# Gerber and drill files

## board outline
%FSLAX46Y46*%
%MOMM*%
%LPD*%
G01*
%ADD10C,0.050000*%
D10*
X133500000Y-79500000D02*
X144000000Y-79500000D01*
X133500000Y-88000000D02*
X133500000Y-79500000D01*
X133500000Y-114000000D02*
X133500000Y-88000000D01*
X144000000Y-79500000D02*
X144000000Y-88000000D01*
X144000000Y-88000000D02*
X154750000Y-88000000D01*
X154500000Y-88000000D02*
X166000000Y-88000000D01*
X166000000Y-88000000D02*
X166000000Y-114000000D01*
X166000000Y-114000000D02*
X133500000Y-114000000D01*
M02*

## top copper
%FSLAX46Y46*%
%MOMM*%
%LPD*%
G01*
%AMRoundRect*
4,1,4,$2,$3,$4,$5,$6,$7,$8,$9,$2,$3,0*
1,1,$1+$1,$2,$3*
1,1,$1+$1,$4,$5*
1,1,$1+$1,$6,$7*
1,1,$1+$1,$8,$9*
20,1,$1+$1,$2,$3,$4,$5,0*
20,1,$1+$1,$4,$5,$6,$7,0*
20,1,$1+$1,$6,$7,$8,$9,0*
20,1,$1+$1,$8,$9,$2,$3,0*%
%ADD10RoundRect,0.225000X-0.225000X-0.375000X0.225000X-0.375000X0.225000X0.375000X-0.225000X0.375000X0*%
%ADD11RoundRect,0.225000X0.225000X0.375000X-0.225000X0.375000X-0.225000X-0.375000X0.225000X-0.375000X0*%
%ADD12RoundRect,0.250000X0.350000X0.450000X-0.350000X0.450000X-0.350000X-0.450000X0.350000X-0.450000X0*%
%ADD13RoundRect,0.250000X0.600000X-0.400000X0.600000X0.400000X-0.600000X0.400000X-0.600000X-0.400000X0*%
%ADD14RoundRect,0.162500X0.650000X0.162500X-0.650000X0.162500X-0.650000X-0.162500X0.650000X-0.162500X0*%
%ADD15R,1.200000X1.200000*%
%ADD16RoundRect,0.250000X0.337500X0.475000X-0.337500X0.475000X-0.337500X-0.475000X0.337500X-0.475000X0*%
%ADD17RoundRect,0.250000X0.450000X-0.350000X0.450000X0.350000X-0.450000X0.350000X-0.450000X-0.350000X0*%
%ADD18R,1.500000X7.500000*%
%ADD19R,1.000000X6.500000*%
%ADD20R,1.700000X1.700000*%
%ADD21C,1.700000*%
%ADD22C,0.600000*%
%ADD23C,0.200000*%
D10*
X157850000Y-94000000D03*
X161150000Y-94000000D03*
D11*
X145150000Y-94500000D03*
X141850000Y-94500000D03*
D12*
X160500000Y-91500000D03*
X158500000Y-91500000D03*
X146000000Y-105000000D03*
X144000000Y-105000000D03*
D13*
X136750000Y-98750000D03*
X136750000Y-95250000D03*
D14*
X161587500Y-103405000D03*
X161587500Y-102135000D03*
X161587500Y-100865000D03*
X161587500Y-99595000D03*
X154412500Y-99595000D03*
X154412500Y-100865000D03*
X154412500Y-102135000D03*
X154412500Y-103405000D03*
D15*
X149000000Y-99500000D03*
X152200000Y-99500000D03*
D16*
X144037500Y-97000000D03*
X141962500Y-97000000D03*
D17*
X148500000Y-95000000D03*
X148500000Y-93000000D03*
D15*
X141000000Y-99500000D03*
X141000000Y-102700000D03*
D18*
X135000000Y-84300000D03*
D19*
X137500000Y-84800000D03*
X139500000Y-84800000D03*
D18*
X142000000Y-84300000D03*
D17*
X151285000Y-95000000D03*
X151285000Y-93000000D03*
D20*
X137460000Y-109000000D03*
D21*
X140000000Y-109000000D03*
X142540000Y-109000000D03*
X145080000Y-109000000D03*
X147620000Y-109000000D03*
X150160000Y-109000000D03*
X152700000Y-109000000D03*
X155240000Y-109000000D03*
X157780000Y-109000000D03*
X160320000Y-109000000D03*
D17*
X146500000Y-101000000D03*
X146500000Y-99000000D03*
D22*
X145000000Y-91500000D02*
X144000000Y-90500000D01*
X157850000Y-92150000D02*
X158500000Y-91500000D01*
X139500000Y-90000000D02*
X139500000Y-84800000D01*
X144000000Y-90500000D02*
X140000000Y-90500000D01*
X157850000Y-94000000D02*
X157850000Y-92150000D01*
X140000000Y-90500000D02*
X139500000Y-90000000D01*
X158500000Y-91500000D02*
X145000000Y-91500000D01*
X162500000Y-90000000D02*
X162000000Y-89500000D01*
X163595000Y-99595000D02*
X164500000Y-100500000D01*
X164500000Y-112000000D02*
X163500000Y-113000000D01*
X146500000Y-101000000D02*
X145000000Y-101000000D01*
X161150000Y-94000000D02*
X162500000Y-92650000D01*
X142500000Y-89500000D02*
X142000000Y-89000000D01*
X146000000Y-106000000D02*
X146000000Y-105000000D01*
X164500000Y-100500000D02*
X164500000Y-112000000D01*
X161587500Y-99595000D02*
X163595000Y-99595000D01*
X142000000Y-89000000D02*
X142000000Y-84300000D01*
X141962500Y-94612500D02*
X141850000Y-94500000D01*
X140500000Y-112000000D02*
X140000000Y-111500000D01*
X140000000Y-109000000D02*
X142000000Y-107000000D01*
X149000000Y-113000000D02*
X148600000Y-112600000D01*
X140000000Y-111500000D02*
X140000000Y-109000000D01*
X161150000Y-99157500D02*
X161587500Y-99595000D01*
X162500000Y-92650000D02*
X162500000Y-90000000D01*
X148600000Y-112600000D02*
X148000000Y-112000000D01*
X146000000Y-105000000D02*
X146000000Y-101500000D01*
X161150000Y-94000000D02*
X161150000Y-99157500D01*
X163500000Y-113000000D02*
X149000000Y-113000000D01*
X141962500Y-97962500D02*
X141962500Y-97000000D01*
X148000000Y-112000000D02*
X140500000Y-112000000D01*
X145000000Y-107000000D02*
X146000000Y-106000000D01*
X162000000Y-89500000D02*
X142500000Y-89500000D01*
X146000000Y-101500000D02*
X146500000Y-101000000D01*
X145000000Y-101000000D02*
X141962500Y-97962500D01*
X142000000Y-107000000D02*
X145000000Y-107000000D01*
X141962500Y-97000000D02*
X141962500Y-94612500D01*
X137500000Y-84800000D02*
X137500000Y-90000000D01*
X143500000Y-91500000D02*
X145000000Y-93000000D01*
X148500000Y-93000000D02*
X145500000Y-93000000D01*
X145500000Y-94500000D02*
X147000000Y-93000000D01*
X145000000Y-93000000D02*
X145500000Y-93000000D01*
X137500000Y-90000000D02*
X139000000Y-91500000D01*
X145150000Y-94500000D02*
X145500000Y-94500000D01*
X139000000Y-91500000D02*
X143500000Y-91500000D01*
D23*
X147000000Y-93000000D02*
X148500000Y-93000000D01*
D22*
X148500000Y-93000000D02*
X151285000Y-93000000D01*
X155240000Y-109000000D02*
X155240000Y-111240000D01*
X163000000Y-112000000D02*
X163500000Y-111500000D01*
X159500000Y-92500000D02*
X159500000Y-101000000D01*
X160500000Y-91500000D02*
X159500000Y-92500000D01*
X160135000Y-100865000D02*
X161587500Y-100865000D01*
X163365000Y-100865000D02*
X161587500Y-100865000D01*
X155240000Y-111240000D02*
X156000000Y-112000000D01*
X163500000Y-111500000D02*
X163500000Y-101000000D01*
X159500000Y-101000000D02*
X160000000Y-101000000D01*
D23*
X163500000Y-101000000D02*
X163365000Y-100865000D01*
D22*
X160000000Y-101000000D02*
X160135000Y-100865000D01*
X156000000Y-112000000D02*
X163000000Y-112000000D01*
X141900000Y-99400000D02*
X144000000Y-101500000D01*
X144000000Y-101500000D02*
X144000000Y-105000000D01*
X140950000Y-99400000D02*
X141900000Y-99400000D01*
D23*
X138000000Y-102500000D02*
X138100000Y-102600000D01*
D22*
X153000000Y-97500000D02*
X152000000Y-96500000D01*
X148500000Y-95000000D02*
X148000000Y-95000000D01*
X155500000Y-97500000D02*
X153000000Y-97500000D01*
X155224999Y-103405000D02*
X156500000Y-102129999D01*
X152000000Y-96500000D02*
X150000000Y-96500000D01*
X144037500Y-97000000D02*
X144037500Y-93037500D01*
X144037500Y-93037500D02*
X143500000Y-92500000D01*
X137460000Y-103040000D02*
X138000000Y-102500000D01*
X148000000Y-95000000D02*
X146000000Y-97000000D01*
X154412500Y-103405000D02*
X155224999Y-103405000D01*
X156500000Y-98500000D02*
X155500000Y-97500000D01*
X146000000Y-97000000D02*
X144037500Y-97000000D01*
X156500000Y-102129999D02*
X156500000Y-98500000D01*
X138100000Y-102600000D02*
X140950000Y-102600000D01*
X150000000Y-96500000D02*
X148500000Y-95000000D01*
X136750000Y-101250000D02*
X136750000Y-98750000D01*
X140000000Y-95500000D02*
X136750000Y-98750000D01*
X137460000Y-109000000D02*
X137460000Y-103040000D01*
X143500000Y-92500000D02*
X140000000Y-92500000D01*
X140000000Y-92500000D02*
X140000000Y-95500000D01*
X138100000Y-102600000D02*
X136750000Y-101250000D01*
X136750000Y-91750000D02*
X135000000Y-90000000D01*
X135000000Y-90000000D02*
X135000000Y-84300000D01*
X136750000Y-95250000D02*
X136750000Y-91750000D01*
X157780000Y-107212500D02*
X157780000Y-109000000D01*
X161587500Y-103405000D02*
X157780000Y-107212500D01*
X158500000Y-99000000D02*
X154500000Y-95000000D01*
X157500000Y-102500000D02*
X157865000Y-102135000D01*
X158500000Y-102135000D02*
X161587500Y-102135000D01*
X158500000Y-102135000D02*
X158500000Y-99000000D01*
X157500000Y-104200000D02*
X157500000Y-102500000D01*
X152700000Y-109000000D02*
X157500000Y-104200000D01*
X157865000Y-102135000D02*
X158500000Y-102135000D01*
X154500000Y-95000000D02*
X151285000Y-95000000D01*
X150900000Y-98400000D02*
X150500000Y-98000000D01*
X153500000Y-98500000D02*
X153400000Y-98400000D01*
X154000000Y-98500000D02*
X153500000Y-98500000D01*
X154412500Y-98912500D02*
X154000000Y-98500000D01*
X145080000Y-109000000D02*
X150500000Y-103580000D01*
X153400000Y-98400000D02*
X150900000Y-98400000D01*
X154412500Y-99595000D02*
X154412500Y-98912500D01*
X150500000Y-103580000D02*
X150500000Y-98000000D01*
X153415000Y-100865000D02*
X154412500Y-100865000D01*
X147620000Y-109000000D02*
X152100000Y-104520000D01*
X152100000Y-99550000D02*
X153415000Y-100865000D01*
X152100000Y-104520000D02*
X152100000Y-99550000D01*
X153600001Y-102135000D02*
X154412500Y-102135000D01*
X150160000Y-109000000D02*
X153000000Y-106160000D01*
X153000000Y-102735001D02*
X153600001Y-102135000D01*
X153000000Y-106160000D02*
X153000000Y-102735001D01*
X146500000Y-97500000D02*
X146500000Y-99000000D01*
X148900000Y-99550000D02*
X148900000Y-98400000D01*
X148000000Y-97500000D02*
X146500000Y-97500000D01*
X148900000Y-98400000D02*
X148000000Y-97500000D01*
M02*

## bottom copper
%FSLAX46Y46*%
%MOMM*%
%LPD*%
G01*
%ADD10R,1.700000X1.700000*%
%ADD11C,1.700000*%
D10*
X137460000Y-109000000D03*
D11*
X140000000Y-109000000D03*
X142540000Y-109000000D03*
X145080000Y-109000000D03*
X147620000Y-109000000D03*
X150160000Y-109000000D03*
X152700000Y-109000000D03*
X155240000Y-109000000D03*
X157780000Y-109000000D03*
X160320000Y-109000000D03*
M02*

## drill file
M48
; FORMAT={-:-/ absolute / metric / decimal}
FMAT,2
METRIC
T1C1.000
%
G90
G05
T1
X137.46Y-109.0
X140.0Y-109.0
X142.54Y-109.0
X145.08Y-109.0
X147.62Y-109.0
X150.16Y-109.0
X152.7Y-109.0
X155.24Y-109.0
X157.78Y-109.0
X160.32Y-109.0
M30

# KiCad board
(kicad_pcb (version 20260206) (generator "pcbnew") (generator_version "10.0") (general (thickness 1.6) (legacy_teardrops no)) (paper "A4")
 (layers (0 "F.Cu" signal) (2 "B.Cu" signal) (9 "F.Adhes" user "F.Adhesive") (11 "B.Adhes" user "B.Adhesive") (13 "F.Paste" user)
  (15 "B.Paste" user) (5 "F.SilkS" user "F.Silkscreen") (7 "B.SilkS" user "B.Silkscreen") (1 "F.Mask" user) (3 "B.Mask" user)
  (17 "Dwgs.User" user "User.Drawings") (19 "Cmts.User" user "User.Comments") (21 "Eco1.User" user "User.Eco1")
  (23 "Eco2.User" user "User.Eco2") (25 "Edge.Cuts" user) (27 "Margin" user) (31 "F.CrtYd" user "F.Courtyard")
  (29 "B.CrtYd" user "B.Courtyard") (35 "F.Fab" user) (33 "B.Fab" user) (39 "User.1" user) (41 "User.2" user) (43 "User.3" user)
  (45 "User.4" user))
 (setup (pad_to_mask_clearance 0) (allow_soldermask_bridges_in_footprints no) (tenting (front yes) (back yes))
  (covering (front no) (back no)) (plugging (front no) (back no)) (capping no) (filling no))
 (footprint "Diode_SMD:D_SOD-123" (layer "F.Cu") (at 159.5 94)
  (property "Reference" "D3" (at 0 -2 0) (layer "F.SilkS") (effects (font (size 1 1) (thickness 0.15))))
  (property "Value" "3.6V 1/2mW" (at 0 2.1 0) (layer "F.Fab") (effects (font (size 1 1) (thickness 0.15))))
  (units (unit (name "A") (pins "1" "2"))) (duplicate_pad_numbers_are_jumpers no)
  (pad "1" smd roundrect (at -1.65 0) (size 0.9 1.2) (layers "F.Cu" "F.Mask" "F.Paste") (roundrect_rratio 0.25) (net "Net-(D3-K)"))
  (pad "2" smd roundrect (at 1.65 0) (size 0.9 1.2) (layers "F.Cu" "F.Mask" "F.Paste") (roundrect_rratio 0.25) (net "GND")))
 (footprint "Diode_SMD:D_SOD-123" (layer "F.Cu") (at 143.5 94.5 180)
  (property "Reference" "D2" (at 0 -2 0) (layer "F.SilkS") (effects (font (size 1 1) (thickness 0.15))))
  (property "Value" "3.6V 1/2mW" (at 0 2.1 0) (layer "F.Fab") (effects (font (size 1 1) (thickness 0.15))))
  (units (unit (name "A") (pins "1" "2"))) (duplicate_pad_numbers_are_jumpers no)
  (pad "1" smd roundrect (at -1.65 0 180) (size 0.9 1.2) (layers "F.Cu" "F.Mask" "F.Paste") (roundrect_rratio 0.25) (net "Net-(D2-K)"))
  (pad "2" smd roundrect (at 1.65 0 180) (size 0.9 1.2) (layers "F.Cu" "F.Mask" "F.Paste") (roundrect_rratio 0.25) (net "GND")))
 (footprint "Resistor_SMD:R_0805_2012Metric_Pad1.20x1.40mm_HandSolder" (layer "F.Cu") (at 159.5 91.5 180)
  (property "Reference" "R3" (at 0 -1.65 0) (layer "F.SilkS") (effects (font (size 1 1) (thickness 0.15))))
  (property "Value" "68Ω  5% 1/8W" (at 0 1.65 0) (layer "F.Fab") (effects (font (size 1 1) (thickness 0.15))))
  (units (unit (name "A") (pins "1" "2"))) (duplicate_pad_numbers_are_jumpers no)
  (pad "1" smd roundrect (at -1 0 180) (size 1.2 1.4) (layers "F.Cu" "F.Mask" "F.Paste") (roundrect_rratio 0.208333) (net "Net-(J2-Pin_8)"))
  (pad "2" smd roundrect (at 1 0 180) (size 1.2 1.4) (layers "F.Cu" "F.Mask" "F.Paste") (roundrect_rratio 0.208333) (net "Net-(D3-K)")))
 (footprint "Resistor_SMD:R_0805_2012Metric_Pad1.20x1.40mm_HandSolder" (layer "F.Cu") (at 145 105 180)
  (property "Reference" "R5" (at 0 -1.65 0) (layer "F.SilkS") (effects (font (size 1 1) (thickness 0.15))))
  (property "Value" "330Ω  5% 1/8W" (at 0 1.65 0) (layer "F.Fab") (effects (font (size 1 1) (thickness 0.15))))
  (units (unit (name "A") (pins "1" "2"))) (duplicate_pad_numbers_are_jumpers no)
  (pad "1" smd roundrect (at -1 0 180) (size 1.2 1.4) (layers "F.Cu" "F.Mask" "F.Paste") (roundrect_rratio 0.208333) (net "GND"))
  (pad "2" smd roundrect (at 1 0 180) (size 1.2 1.4) (layers "F.Cu" "F.Mask" "F.Paste") (roundrect_rratio 0.208333) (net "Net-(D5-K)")))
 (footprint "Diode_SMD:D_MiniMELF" (layer "F.Cu") (at 136.75 97 90)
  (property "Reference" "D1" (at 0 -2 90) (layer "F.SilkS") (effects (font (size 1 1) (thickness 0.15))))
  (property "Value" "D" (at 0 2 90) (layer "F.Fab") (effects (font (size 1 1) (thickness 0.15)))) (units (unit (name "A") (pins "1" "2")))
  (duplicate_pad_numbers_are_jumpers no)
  (pad "1" smd roundrect (at -1.75 0 90) (size 1.3 1.7) (layers "F.Cu" "F.Mask" "F.Paste") (roundrect_rratio 0.1923076923) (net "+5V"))
  (pad "2" smd roundrect (at 1.75 0 90) (size 1.3 1.7) (layers "F.Cu" "F.Mask" "F.Paste") (roundrect_rratio 0.1923076923) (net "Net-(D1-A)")))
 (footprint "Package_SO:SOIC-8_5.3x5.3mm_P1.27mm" (layer "F.Cu") (at 158 101.5 180)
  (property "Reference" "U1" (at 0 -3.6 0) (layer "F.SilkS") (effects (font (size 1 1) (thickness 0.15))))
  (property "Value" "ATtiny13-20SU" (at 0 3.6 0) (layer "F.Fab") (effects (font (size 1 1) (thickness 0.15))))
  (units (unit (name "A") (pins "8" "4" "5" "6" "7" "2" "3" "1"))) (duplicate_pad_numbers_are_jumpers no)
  (pad "1" smd roundrect (at -3.5875 -1.905 180) (size 1.625 0.65) (layers "F.Cu" "F.Mask" "F.Paste") (roundrect_rratio 0.25)
   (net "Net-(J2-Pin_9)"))
  (pad "2" smd roundrect (at -3.5875 -0.635 180) (size 1.625 0.65) (layers "F.Cu" "F.Mask" "F.Paste") (roundrect_rratio 0.25)
   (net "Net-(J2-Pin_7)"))
  (pad "3" smd roundrect (at -3.5875 0.635 180) (size 1.625 0.65) (layers "F.Cu" "F.Mask" "F.Paste") (roundrect_rratio 0.25)
   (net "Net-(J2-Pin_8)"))
  (pad "4" smd roundrect (at -3.5875 1.905 180) (size 1.625 0.65) (layers "F.Cu" "F.Mask" "F.Paste") (roundrect_rratio 0.25) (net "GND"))
  (pad "5" smd roundrect (at 3.5875 1.905 180) (size 1.625 0.65) (layers "F.Cu" "F.Mask" "F.Paste") (roundrect_rratio 0.25)
   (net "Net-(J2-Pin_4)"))
  (pad "6" smd roundrect (at 3.5875 0.635 180) (size 1.625 0.65) (layers "F.Cu" "F.Mask" "F.Paste") (roundrect_rratio 0.25)
   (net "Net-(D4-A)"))
  (pad "7" smd roundrect (at 3.5875 -0.635 180) (size 1.625 0.65) (layers "F.Cu" "F.Mask" "F.Paste") (roundrect_rratio 0.25)
   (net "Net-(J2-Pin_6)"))
  (pad "8" smd roundrect (at 3.5875 -1.905 180) (size 1.625 0.65) (layers "F.Cu" "F.Mask" "F.Paste") (roundrect_rratio 0.25) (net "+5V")))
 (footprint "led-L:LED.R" (layer "F.Cu") (at 142.98 93.469999)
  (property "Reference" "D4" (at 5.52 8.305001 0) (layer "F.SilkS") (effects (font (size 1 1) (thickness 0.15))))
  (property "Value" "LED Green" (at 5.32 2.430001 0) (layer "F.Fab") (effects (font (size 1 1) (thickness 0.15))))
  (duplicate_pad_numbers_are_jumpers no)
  (pad "1" smd rect (at 6.02 6.030001) (size 1.2 1.2) (layers "F.Cu" "F.Mask" "F.Paste") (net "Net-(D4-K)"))
  (pad "2" smd rect (at 9.22 6.030001) (size 1.2 1.2) (layers "F.Cu" "F.Mask" "F.Paste") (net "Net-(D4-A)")))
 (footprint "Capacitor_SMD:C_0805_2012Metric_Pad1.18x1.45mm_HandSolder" (layer "F.Cu") (at 143 97 180)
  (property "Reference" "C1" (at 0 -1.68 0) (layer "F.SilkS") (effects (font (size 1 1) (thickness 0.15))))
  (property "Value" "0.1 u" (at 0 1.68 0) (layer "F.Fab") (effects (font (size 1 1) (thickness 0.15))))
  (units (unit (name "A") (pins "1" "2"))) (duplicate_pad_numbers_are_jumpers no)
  (pad "1" smd roundrect (at -1.0375 0 180) (size 1.175 1.45) (layers "F.Cu" "F.Mask" "F.Paste") (roundrect_rratio 0.212766) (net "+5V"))
  (pad "2" smd roundrect (at 1.0375 0 180) (size 1.175 1.45) (layers "F.Cu" "F.Mask" "F.Paste") (roundrect_rratio 0.212766) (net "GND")))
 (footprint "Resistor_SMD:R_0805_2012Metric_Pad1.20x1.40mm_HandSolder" (layer "F.Cu") (at 148.5 94 90)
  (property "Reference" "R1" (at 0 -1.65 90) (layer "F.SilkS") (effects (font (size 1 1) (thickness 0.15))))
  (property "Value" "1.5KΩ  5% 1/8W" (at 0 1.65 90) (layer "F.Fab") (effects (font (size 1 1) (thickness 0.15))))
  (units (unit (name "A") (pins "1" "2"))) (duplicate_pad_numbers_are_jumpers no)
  (pad "1" smd roundrect (at -1 0 90) (size 1.2 1.4) (layers "F.Cu" "F.Mask" "F.Paste") (roundrect_rratio 0.208333) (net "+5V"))
  (pad "2" smd roundrect (at 1 0 90) (size 1.2 1.4) (layers "F.Cu" "F.Mask" "F.Paste") (roundrect_rratio 0.208333) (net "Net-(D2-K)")))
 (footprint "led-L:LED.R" (layer "F.Cu") (at 146.08 96.168469 -90)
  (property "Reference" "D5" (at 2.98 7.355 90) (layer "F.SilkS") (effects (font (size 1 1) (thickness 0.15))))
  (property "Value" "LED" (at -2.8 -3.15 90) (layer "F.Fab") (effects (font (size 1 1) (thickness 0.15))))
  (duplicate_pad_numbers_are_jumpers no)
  (pad "1" smd rect (at 3.331531 5.08 270) (size 1.2 1.2) (layers "F.Cu" "F.Mask" "F.Paste") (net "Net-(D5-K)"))
  (pad "2" smd rect (at 6.531531 5.08 270) (size 1.2 1.2) (layers "F.Cu" "F.Mask" "F.Paste") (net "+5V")))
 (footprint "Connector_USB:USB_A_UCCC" (layer "F.Cu") (at 138.5 84.5 -90)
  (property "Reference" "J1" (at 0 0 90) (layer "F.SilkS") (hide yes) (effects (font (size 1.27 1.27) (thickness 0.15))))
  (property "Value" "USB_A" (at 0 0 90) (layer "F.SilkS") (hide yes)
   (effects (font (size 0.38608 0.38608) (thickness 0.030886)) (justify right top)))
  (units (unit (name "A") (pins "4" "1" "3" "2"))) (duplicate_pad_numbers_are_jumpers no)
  (pad "1" smd rect (at -0.2 3.5 270) (size 7.5 1.5) (layers "F.Cu" "F.Mask" "F.Paste") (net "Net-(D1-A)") (solder_mask_margin 0.1016))
  (pad "2" smd rect (at 0.3 1 270) (size 6.5 1) (layers "F.Cu" "F.Mask" "F.Paste") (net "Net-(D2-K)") (solder_mask_margin 0.1016))
  (pad "3" smd rect (at 0.3 -1 270) (size 6.5 1) (layers "F.Cu" "F.Mask" "F.Paste") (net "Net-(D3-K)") (solder_mask_margin 0.1016))
  (pad "4" smd rect (at -0.2 -3.5 270) (size 7.5 1.5) (layers "F.Cu" "F.Mask" "F.Paste") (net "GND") (solder_mask_margin 0.1016)))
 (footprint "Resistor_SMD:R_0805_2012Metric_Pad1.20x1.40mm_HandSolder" (layer "F.Cu") (at 151.285 94 90)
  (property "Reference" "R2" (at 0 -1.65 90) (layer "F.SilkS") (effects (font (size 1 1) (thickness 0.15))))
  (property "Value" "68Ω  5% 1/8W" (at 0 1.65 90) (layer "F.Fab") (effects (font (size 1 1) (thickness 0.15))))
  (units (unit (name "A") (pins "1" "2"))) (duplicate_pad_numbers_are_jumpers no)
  (pad "1" smd roundrect (at -1 0 90) (size 1.2 1.4) (layers "F.Cu" "F.Mask" "F.Paste") (roundrect_rratio 0.208333) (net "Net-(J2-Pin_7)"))
  (pad "2" smd roundrect (at 1 0 90) (size 1.2 1.4) (layers "F.Cu" "F.Mask" "F.Paste") (roundrect_rratio 0.208333) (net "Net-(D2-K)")))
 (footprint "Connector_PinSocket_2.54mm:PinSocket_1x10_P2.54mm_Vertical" (layer "F.Cu") (at 137.46 109 90)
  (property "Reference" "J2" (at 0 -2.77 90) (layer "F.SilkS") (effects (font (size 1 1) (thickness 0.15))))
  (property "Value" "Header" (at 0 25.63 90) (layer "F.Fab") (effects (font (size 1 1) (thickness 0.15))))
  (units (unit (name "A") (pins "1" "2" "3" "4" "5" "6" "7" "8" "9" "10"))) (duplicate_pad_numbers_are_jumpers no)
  (pad "1" thru_hole rect (at 0 0 90) (size 1.7 1.7) (drill 1) (layers "*.Cu" "*.Mask") (remove_unused_layers no) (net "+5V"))
  (pad "2" thru_hole circle (at 0 2.54 90) (size 1.7 1.7) (drill 1) (layers "*.Cu" "*.Mask") (remove_unused_layers no) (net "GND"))
  (pad "3" thru_hole circle (at 0 5.08 90) (size 1.7 1.7) (drill 1) (layers "*.Cu" "*.Mask") (remove_unused_layers no)
   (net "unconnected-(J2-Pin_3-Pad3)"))
  (pad "4" thru_hole circle (at 0 7.62 90) (size 1.7 1.7) (drill 1) (layers "*.Cu" "*.Mask") (remove_unused_layers no)
   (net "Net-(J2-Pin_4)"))
  (pad "5" thru_hole circle (at 0 10.16 90) (size 1.7 1.7) (drill 1) (layers "*.Cu" "*.Mask") (remove_unused_layers no) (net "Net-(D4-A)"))
  (pad "6" thru_hole circle (at 0 12.7 90) (size 1.7 1.7) (drill 1) (layers "*.Cu" "*.Mask") (remove_unused_layers no)
   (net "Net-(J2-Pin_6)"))
  (pad "7" thru_hole circle (at 0 15.24 90) (size 1.7 1.7) (drill 1) (layers "*.Cu" "*.Mask") (remove_unused_layers no)
   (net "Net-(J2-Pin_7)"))
  (pad "8" thru_hole circle (at 0 17.78 90) (size 1.7 1.7) (drill 1) (layers "*.Cu" "*.Mask") (remove_unused_layers no)
   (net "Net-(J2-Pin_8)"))
  (pad "9" thru_hole circle (at 0 20.32 90) (size 1.7 1.7) (drill 1) (layers "*.Cu" "*.Mask") (remove_unused_layers no)
   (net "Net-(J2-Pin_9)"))
  (pad "10" thru_hole circle (at 0 22.86 90) (size 1.7 1.7) (drill 1) (layers "*.Cu" "*.Mask") (remove_unused_layers no)
   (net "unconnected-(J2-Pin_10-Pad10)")))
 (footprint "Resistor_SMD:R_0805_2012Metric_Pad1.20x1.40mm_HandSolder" (layer "F.Cu") (at 146.5 100 90)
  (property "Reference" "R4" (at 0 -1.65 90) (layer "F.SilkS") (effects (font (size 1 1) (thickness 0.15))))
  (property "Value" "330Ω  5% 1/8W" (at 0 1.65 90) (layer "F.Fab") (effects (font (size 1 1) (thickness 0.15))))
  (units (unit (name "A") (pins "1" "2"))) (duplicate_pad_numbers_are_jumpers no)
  (pad "1" smd roundrect (at -1 0 90) (size 1.2 1.4) (layers "F.Cu" "F.Mask" "F.Paste") (roundrect_rratio 0.208333) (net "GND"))
  (pad "2" smd roundrect (at 1 0 90) (size 1.2 1.4) (layers "F.Cu" "F.Mask" "F.Paste") (roundrect_rratio 0.208333) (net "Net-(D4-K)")))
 (gr_line (start 133.5 79.5) (end 144 79.5) (stroke (width 0.05) (type default)) (layer "Edge.Cuts"))
 (gr_line (start 133.5 88) (end 133.5 79.5) (stroke (width 0.05) (type default)) (layer "Edge.Cuts"))
 (gr_line (start 133.5 114) (end 133.5 88) (stroke (width 0.05) (type default)) (layer "Edge.Cuts"))
 (gr_line (start 144 79.5) (end 144 88) (stroke (width 0.05) (type default)) (layer "Edge.Cuts"))
 (gr_line (start 144 88) (end 154.75 88) (stroke (width 0.05) (type default)) (layer "Edge.Cuts"))
 (gr_line (start 154.5 88) (end 166 88) (stroke (width 0.05) (type default)) (layer "Edge.Cuts"))
 (gr_line (start 166 88) (end 166 114) (stroke (width 0.05) (type default)) (layer "Edge.Cuts"))
 (gr_line (start 166 114) (end 133.5 114) (stroke (width 0.05) (type default)) (layer "Edge.Cuts"))
 (segment (start 145 91.5) (end 144 90.5) (width 0.6) (layer "F.Cu") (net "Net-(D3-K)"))
 (segment (start 157.85 92.15) (end 158.5 91.5) (width 0.6) (layer "F.Cu") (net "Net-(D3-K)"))
 (segment (start 139.5 90) (end 139.5 84.8) (width 0.6) (layer "F.Cu") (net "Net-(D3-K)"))
 (segment (start 144 90.5) (end 140 90.5) (width 0.6) (layer "F.Cu") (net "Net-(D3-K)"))
 (segment (start 157.85 94) (end 157.85 92.15) (width 0.6) (layer "F.Cu") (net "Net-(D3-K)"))
 (segment (start 140 90.5) (end 139.5 90) (width 0.6) (layer "F.Cu") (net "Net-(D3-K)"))
 (segment (start 158.5 91.5) (end 145 91.5) (width 0.6) (layer "F.Cu") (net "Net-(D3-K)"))
 (segment (start 162.5 90) (end 162 89.5) (width 0.6) (layer "F.Cu") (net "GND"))
 (segment (start 163.595 99.595) (end 164.5 100.5) (width 0.6) (layer "F.Cu") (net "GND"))
 (segment (start 164.5 112) (end 163.5 113) (width 0.6) (layer "F.Cu") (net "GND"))
 (segment (start 146.5 101) (end 145 101) (width 0.6) (layer "F.Cu") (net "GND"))
 (segment (start 161.15 94) (end 162.5 92.65) (width 0.6) (layer "F.Cu") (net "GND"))
 (segment (start 142.5 89.5) (end 142 89) (width 0.6) (layer "F.Cu") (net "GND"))
 (segment (start 146 106) (end 146 105) (width 0.6) (layer "F.Cu") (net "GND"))
 (segment (start 164.5 100.5) (end 164.5 112) (width 0.6) (layer "F.Cu") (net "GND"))
 (segment (start 161.5875 99.595) (end 163.595 99.595) (width 0.6) (layer "F.Cu") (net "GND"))
 (segment (start 142 89) (end 142 84.3) (width 0.6) (layer "F.Cu") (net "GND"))
 (segment (start 141.9625 94.6125) (end 141.85 94.5) (width 0.6) (layer "F.Cu") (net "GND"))
 (segment (start 140.5 112) (end 140 111.5) (width 0.6) (layer "F.Cu") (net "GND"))
 (segment (start 140 109) (end 142 107) (width 0.6) (layer "F.Cu") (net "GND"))
 (segment (start 149 113) (end 148.6 112.6) (width 0.6) (layer "F.Cu") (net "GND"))
 (segment (start 140 111.5) (end 140 109) (width 0.6) (layer "F.Cu") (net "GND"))
 (segment (start 161.15 99.1575) (end 161.5875 99.595) (width 0.6) (layer "F.Cu") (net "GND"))
 (segment (start 162.5 92.65) (end 162.5 90) (width 0.6) (layer "F.Cu") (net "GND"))
 (segment (start 148.6 112.6) (end 148 112) (width 0.6) (layer "F.Cu") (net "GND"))
 (segment (start 146 105) (end 146 101.5) (width 0.6) (layer "F.Cu") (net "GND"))
 (segment (start 161.15 94) (end 161.15 99.1575) (width 0.6) (layer "F.Cu") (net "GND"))
 (segment (start 163.5 113) (end 149 113) (width 0.6) (layer "F.Cu") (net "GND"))
 (segment (start 141.9625 97.9625) (end 141.9625 97) (width 0.6) (layer "F.Cu") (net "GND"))
 (segment (start 148 112) (end 140.5 112) (width 0.6) (layer "F.Cu") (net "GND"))
 (segment (start 145 107) (end 146 106) (width 0.6) (layer "F.Cu") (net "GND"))
 (segment (start 162 89.5) (end 142.5 89.5) (width 0.6) (layer "F.Cu") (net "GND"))
 (segment (start 146 101.5) (end 146.5 101) (width 0.6) (layer "F.Cu") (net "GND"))
 (segment (start 145 101) (end 141.9625 97.9625) (width 0.6) (layer "F.Cu") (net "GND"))
 (segment (start 142 107) (end 145 107) (width 0.6) (layer "F.Cu") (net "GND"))
 (segment (start 141.9625 97) (end 141.9625 94.6125) (width 0.6) (layer "F.Cu") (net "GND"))
 (segment (start 137.5 84.8) (end 137.5 90) (width 0.6) (layer "F.Cu") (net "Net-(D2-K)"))
 (segment (start 143.5 91.5) (end 145 93) (width 0.6) (layer "F.Cu") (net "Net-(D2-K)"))
 (segment (start 148.5 93) (end 145.5 93) (width 0.6) (layer "F.Cu") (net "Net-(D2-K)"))
 (segment (start 145.5 94.5) (end 147 93) (width 0.6) (layer "F.Cu") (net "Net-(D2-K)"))
 (segment (start 145 93) (end 145.5 93) (width 0.6) (layer "F.Cu") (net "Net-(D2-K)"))
 (segment (start 137.5 90) (end 139 91.5) (width 0.6) (layer "F.Cu") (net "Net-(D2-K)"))
 (segment (start 145.15 94.5) (end 145.5 94.5) (width 0.6) (layer "F.Cu") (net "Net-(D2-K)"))
 (segment (start 139 91.5) (end 143.5 91.5) (width 0.6) (layer "F.Cu") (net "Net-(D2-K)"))
 (segment (start 147 93) (end 148.5 93) (width 0.2) (layer "F.Cu") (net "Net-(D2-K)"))
 (segment (start 148.5 93) (end 151.285 93) (width 0.6) (layer "F.Cu") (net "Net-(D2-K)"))
 (segment (start 155.24 109) (end 155.24 111.24) (width 0.6) (layer "F.Cu") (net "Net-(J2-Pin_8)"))
 (segment (start 163 112) (end 163.5 111.5) (width 0.6) (layer "F.Cu") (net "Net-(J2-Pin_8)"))
 (segment (start 159.5 92.5) (end 159.5 101) (width 0.6) (layer "F.Cu") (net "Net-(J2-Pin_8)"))
 (segment (start 160.5 91.5) (end 159.5 92.5) (width 0.6) (layer "F.Cu") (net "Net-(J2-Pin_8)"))
 (segment (start 160.135 100.865) (end 161.5875 100.865) (width 0.6) (layer "F.Cu") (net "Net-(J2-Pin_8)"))
 (segment (start 163.365 100.865) (end 161.5875 100.865) (width 0.6) (layer "F.Cu") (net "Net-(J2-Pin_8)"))
 (segment (start 155.24 111.24) (end 156 112) (width 0.6) (layer "F.Cu") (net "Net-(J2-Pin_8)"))
 (segment (start 163.5 111.5) (end 163.5 101) (width 0.6) (layer "F.Cu") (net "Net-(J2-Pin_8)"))
 (segment (start 159.5 101) (end 160 101) (width 0.6) (layer "F.Cu") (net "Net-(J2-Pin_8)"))
 (segment (start 163.5 101) (end 163.365 100.865) (width 0.2) (layer "F.Cu") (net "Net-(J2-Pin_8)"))
 (segment (start 160 101) (end 160.135 100.865) (width 0.6) (layer "F.Cu") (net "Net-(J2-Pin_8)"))
 (segment (start 156 112) (end 163 112) (width 0.6) (layer "F.Cu") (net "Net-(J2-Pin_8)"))
 (segment (start 141.9 99.4) (end 144 101.5) (width 0.6) (layer "F.Cu") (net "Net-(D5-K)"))
 (segment (start 144 101.5) (end 144 105) (width 0.6) (layer "F.Cu") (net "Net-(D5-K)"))
 (segment (start 140.95 99.4) (end 141.9 99.4) (width 0.6) (layer "F.Cu") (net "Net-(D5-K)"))
 (segment (start 138 102.5) (end 138.1 102.6) (width 0.2) (layer "F.Cu") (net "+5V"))
 (segment (start 153 97.5) (end 152 96.5) (width 0.6) (layer "F.Cu") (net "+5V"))
 (segment (start 148.5 95) (end 148 95) (width 0.6) (layer "F.Cu") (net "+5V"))
 (segment (start 155.5 97.5) (end 153 97.5) (width 0.6) (layer "F.Cu") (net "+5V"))
 (segment (start 155.224999 103.405) (end 156.5 102.129999) (width 0.6) (layer "F.Cu") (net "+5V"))
 (segment (start 152 96.5) (end 150 96.5) (width 0.6) (layer "F.Cu") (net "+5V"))
 (segment (start 144.0375 97) (end 144.0375 93.0375) (width 0.6) (layer "F.Cu") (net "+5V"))
 (segment (start 144.0375 93.0375) (end 143.5 92.5) (width 0.6) (layer "F.Cu") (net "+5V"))
 (segment (start 137.46 103.04) (end 138 102.5) (width 0.6) (layer "F.Cu") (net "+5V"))
 (segment (start 148 95) (end 146 97) (width 0.6) (layer "F.Cu") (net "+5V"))
 (segment (start 154.4125 103.405) (end 155.224999 103.405) (width 0.6) (layer "F.Cu") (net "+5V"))
 (segment (start 156.5 98.5) (end 155.5 97.5) (width 0.6) (layer "F.Cu") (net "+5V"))
 (segment (start 146 97) (end 144.0375 97) (width 0.6) (layer "F.Cu") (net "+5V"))
 (segment (start 156.5 102.129999) (end 156.5 98.5) (width 0.6) (layer "F.Cu") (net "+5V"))
 (segment (start 138.1 102.6) (end 140.95 102.6) (width 0.6) (layer "F.Cu") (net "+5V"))
 (segment (start 150 96.5) (end 148.5 95) (width 0.6) (layer "F.Cu") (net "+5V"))
 (segment (start 136.75 101.25) (end 136.75 98.75) (width 0.6) (layer "F.Cu") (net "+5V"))
 (segment (start 140 95.5) (end 136.75 98.75) (width 0.6) (layer "F.Cu") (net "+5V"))
 (segment (start 137.46 109) (end 137.46 103.04) (width 0.6) (layer "F.Cu") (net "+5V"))
 (segment (start 143.5 92.5) (end 140 92.5) (width 0.6) (layer "F.Cu") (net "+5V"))
 (segment (start 140 92.5) (end 140 95.5) (width 0.6) (layer "F.Cu") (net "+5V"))
 (segment (start 138.1 102.6) (end 136.75 101.25) (width 0.6) (layer "F.Cu") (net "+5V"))
 (segment (start 136.75 91.75) (end 135 90) (width 0.6) (layer "F.Cu") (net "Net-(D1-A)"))
 (segment (start 135 90) (end 135 84.3) (width 0.6) (layer "F.Cu") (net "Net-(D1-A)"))
 (segment (start 136.75 95.25) (end 136.75 91.75) (width 0.6) (layer "F.Cu") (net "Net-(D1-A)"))
 (segment (start 157.78 107.2125) (end 157.78 109) (width 0.6) (layer "F.Cu") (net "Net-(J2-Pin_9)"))
 (segment (start 161.5875 103.405) (end 157.78 107.2125) (width 0.6) (layer "F.Cu") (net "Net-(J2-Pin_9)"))
 (segment (start 158.5 99) (end 154.5 95) (width 0.6) (layer "F.Cu") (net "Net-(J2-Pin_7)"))
 (segment (start 157.5 102.5) (end 157.865 102.135) (width 0.6) (layer "F.Cu") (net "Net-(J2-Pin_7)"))
 (segment (start 158.5 102.135) (end 161.5875 102.135) (width 0.6) (layer "F.Cu") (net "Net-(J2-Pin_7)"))
 (segment (start 158.5 102.135) (end 158.5 99) (width 0.6) (layer "F.Cu") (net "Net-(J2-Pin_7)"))
 (segment (start 157.5 104.2) (end 157.5 102.5) (width 0.6) (layer "F.Cu") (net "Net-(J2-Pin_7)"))
 (segment (start 152.7 109) (end 157.5 104.2) (width 0.6) (layer "F.Cu") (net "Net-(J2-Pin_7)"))
 (segment (start 157.865 102.135) (end 158.5 102.135) (width 0.6) (layer "F.Cu") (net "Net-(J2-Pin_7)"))
 (segment (start 154.5 95) (end 151.285 95) (width 0.6) (layer "F.Cu") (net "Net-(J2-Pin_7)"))
 (segment (start 150.9 98.4) (end 150.5 98) (width 0.6) (layer "F.Cu") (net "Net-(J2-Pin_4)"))
 (segment (start 153.5 98.5) (end 153.4 98.4) (width 0.6) (layer "F.Cu") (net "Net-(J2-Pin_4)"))
 (segment (start 154 98.5) (end 153.5 98.5) (width 0.6) (layer "F.Cu") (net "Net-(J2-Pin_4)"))
 (segment (start 154.4125 98.9125) (end 154 98.5) (width 0.6) (layer "F.Cu") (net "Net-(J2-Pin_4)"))
 (segment (start 145.08 109) (end 150.5 103.58) (width 0.6) (layer "F.Cu") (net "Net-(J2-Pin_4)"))
 (segment (start 153.4 98.4) (end 150.9 98.4) (width 0.6) (layer "F.Cu") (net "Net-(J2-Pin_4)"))
 (segment (start 154.4125 99.595) (end 154.4125 98.9125) (width 0.6) (layer "F.Cu") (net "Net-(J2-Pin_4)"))
 (segment (start 150.5 103.58) (end 150.5 98) (width 0.6) (layer "F.Cu") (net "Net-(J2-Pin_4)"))
 (segment (start 153.415 100.865) (end 154.4125 100.865) (width 0.6) (layer "F.Cu") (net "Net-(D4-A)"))
 (segment (start 147.62 109) (end 152.1 104.52) (width 0.6) (layer "F.Cu") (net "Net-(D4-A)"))
 (segment (start 152.1 99.55) (end 153.415 100.865) (width 0.6) (layer "F.Cu") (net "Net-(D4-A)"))
 (segment (start 152.1 104.52) (end 152.1 99.55) (width 0.6) (layer "F.Cu") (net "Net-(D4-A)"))
 (segment (start 153.600001 102.135) (end 154.4125 102.135) (width 0.6) (layer "F.Cu") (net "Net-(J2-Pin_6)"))
 (segment (start 150.16 109) (end 153 106.16) (width 0.6) (layer "F.Cu") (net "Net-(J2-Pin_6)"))
 (segment (start 153 102.735001) (end 153.600001 102.135) (width 0.6) (layer "F.Cu") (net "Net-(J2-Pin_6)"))
 (segment (start 153 106.16) (end 153 102.735001) (width 0.6) (layer "F.Cu") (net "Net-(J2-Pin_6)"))
 (segment (start 146.5 97.5) (end 146.5 99) (width 0.6) (layer "F.Cu") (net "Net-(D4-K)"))
 (segment (start 148.9 99.55) (end 148.9 98.4) (width 0.6) (layer "F.Cu") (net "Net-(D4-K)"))
 (segment (start 148 97.5) (end 146.5 97.5) (width 0.6) (layer "F.Cu") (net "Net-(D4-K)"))
 (segment (start 148.9 98.4) (end 148 97.5) (width 0.6) (layer "F.Cu") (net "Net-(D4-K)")))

